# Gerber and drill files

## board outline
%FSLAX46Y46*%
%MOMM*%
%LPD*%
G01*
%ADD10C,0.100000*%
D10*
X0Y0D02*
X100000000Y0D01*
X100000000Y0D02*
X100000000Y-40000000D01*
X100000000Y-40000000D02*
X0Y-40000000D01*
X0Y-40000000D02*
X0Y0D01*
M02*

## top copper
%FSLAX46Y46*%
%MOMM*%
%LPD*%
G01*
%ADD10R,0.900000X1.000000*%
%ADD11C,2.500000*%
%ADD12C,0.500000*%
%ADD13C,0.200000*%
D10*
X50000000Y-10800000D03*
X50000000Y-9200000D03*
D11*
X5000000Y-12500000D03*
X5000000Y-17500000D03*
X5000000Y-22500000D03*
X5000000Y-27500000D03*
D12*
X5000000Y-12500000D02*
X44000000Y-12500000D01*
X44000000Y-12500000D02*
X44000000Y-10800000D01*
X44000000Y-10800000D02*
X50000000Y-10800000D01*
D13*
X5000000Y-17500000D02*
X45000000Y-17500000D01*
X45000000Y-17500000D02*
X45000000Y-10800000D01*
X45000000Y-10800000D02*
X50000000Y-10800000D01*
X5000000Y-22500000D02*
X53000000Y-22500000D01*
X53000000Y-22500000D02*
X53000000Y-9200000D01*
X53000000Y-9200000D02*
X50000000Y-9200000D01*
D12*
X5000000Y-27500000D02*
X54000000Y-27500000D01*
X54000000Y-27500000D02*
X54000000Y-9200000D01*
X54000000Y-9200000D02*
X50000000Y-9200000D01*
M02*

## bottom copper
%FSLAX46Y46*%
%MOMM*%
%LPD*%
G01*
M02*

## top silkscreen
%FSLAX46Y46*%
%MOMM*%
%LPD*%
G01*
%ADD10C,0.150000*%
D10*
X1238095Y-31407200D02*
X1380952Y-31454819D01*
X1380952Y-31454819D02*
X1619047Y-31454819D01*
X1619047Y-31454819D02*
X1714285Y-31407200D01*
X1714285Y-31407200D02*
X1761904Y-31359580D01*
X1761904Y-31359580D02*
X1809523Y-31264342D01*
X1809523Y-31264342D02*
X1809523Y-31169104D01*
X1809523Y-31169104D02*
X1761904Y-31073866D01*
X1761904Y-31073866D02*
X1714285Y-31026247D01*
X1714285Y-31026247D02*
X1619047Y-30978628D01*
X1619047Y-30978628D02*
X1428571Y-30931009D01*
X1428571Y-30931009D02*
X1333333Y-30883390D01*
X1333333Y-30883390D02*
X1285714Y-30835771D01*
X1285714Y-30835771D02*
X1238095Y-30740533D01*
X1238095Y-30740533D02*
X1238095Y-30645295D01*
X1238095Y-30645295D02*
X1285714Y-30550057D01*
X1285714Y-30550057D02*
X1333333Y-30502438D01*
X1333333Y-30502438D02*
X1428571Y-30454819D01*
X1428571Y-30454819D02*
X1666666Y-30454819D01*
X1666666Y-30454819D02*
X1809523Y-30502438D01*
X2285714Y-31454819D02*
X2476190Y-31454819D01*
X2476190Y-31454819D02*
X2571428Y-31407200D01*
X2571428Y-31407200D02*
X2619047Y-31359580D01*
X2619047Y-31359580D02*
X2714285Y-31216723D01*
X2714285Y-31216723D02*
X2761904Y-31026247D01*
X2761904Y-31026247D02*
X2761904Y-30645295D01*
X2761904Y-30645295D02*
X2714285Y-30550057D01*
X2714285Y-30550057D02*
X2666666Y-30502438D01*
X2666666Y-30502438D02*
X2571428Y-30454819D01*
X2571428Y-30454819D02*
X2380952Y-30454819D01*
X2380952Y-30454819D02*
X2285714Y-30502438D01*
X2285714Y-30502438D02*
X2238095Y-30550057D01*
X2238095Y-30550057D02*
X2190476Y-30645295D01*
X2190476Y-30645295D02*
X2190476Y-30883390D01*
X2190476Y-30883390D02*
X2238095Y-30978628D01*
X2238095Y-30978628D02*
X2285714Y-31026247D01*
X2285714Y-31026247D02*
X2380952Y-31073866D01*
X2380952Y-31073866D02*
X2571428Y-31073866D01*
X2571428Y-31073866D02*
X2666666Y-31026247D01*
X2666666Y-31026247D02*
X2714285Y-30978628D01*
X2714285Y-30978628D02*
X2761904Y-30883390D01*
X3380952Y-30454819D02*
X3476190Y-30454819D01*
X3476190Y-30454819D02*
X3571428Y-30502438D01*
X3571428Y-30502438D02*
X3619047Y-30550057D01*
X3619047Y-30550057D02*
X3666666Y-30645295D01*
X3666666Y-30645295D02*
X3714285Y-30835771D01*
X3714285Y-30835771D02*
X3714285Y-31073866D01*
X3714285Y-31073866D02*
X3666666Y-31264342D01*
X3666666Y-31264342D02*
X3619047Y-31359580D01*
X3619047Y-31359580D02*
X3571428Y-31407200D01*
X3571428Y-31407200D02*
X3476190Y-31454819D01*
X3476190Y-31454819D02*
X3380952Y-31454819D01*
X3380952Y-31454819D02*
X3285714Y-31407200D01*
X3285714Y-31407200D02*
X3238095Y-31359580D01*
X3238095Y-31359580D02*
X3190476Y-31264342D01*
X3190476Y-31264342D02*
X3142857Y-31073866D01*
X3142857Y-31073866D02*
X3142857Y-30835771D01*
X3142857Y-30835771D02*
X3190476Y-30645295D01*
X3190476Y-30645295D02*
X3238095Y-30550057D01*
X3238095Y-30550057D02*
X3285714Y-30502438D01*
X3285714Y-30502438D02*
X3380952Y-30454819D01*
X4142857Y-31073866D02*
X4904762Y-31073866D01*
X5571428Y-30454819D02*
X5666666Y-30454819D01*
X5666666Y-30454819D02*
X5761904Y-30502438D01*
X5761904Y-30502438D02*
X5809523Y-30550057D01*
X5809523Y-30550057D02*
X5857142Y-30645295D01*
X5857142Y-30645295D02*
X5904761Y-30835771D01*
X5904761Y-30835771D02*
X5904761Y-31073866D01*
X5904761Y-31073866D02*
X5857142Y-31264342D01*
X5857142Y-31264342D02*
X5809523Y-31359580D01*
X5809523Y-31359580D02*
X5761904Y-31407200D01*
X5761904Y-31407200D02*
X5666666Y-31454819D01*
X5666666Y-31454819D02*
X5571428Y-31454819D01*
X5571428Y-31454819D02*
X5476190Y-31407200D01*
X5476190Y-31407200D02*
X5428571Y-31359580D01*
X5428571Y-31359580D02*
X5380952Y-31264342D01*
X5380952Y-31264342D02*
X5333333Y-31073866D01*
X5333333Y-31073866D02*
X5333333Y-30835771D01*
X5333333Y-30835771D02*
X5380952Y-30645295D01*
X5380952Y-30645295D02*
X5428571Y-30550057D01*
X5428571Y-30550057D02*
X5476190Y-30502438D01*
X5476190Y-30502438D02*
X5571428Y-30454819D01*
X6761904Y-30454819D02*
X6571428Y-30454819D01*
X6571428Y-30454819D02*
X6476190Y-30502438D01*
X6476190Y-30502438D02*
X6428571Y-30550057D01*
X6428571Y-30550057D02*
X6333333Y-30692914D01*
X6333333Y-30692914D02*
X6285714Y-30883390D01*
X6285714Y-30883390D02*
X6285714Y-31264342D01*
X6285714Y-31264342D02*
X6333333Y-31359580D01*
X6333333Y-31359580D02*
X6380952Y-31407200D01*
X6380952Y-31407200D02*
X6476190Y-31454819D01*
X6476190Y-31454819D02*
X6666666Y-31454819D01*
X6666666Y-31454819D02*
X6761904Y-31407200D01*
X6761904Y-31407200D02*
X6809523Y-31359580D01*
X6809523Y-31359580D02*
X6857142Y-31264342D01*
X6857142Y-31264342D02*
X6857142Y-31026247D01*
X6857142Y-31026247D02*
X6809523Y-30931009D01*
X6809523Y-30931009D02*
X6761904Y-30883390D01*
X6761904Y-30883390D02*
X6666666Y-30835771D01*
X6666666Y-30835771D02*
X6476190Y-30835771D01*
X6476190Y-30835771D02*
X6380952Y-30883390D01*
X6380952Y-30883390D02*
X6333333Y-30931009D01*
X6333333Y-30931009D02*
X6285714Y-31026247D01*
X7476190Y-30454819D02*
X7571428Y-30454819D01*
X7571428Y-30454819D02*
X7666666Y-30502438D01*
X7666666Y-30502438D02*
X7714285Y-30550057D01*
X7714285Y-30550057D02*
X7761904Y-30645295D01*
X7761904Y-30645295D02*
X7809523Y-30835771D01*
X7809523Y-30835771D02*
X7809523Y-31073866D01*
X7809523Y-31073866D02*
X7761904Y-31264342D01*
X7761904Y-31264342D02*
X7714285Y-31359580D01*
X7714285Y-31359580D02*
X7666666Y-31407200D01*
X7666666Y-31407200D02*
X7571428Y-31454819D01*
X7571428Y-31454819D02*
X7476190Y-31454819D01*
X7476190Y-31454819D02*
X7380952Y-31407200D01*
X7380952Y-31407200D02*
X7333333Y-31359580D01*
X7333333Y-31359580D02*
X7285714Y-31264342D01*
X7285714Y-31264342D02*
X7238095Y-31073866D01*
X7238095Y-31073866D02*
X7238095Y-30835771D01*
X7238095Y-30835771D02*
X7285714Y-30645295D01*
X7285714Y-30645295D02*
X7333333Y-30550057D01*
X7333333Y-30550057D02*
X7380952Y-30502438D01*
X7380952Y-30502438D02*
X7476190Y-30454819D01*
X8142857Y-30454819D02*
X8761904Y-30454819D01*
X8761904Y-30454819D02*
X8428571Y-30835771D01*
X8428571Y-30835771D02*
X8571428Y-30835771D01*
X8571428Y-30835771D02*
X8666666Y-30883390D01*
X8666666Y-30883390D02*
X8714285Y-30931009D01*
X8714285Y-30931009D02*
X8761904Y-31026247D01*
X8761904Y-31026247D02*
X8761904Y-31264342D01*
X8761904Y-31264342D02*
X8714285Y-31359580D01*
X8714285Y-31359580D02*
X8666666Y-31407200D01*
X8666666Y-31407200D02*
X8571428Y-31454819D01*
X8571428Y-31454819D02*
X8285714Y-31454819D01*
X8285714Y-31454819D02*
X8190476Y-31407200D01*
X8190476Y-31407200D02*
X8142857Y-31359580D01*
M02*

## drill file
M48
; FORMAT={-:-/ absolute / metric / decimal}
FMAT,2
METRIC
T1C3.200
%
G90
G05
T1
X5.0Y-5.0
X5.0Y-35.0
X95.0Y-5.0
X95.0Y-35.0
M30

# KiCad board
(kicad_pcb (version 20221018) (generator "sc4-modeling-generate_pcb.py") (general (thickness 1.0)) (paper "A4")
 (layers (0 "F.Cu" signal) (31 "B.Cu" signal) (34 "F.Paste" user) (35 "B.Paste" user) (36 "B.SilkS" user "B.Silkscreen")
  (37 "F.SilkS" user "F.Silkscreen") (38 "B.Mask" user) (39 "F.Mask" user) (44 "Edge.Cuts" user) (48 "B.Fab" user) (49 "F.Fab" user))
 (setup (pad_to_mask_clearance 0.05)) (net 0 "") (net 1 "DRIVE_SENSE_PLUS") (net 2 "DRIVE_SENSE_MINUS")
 (gr_line (start 0.0 0.0) (end 100.0 0.0) (layer "Edge.Cuts") (width 0.1))
 (gr_line (start 100.0 0.0) (end 100.0 40.0) (layer "Edge.Cuts") (width 0.1))
 (gr_line (start 100.0 40.0) (end 0.0 40.0) (layer "Edge.Cuts") (width 0.1))
 (gr_line (start 0.0 40.0) (end 0.0 0.0) (layer "Edge.Cuts") (width 0.1))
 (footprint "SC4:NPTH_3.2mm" (layer "F.Cu") (at 5.0 5.0)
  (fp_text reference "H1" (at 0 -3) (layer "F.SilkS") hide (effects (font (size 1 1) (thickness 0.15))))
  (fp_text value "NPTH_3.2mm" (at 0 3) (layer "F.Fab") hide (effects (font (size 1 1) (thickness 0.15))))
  (pad "1" np_thru_hole circle (at 0 0) (size 3.2 3.2) (drill 3.2) (layers "*.Cu" "*.Mask")))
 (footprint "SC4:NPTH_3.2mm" (layer "F.Cu") (at 95.0 5.0)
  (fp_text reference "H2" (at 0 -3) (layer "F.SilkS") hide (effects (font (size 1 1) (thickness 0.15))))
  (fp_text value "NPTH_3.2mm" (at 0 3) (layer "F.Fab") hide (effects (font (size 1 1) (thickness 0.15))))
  (pad "1" np_thru_hole circle (at 0 0) (size 3.2 3.2) (drill 3.2) (layers "*.Cu" "*.Mask")))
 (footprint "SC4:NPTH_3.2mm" (layer "F.Cu") (at 5.0 35.0)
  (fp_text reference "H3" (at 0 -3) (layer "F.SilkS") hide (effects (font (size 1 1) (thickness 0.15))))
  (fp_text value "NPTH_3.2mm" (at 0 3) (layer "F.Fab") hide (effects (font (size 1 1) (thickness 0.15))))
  (pad "1" np_thru_hole circle (at 0 0) (size 3.2 3.2) (drill 3.2) (layers "*.Cu" "*.Mask")))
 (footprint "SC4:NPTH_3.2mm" (layer "F.Cu") (at 95.0 35.0)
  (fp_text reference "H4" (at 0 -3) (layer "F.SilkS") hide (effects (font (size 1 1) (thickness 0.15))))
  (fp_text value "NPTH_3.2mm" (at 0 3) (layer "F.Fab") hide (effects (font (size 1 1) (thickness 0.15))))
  (pad "1" np_thru_hole circle (at 0 0) (size 3.2 3.2) (drill 3.2) (layers "*.Cu" "*.Mask")))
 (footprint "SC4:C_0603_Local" (layer "F.Cu") (at 50.0 10.0 90)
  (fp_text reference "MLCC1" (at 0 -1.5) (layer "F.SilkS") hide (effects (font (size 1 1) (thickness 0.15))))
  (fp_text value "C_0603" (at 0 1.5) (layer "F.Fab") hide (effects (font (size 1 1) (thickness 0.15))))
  (pad "1" smd rect (at -0.8 0) (size 0.9 1.0) (layers "F.Cu" "F.Paste" "F.Mask") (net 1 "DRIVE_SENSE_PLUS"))
  (pad "2" smd rect (at 0.8 0) (size 0.9 1.0) (layers "F.Cu" "F.Paste" "F.Mask") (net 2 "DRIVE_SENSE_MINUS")))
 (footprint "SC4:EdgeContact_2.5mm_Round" (layer "F.Cu") (at 5.0 12.5)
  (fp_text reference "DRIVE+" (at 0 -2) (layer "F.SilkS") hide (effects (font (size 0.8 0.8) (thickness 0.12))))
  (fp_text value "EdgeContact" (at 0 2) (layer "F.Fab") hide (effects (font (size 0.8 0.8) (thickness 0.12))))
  (pad "1" smd circle (at 0 0) (size 2.5 2.5) (layers "F.Cu" "F.Mask") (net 1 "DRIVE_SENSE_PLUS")))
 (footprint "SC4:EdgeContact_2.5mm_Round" (layer "F.Cu") (at 5.0 17.5)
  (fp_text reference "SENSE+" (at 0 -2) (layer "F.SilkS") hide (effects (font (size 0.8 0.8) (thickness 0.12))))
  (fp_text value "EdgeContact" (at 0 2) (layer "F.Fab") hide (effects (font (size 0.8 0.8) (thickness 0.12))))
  (pad "1" smd circle (at 0 0) (size 2.5 2.5) (layers "F.Cu" "F.Mask") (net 1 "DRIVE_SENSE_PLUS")))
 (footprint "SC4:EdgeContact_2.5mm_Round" (layer "F.Cu") (at 5.0 22.5)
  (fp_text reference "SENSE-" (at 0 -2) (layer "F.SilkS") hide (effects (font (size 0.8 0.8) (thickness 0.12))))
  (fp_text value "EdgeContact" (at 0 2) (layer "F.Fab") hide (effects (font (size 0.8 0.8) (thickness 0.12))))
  (pad "1" smd circle (at 0 0) (size 2.5 2.5) (layers "F.Cu" "F.Mask") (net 2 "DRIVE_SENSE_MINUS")))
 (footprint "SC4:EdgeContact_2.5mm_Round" (layer "F.Cu") (at 5.0 27.5)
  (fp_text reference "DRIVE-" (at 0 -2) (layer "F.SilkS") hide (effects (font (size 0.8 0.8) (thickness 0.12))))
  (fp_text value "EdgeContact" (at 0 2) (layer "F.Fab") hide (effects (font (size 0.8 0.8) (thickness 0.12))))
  (pad "1" smd circle (at 0 0) (size 2.5 2.5) (layers "F.Cu" "F.Mask") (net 2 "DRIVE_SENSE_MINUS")))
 (segment (start 5.0 12.5) (end 44.0 12.5) (width 0.5) (layer "F.Cu") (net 1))
 (segment (start 44.0 12.5) (end 44.0 10.8) (width 0.5) (layer "F.Cu") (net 1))
 (segment (start 44.0 10.8) (end 50.0 10.8) (width 0.5) (layer "F.Cu") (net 1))
 (segment (start 5.0 17.5) (end 45.0 17.5) (width 0.2) (layer "F.Cu") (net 1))
 (segment (start 45.0 17.5) (end 45.0 10.8) (width 0.2) (layer "F.Cu") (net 1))
 (segment (start 45.0 10.8) (end 50.0 10.8) (width 0.2) (layer "F.Cu") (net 1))
 (segment (start 5.0 22.5) (end 53.0 22.5) (width 0.2) (layer "F.Cu") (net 2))
 (segment (start 53.0 22.5) (end 53.0 9.2) (width 0.2) (layer "F.Cu") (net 2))
 (segment (start 53.0 9.2) (end 50.0 9.2) (width 0.2) (layer "F.Cu") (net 2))
 (segment (start 5.0 27.5) (end 54.0 27.5) (width 0.5) (layer "F.Cu") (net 2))
 (segment (start 54.0 27.5) (end 54.0 9.2) (width 0.5) (layer "F.Cu") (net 2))
 (segment (start 54.0 9.2) (end 50.0 9.2) (width 0.5) (layer "F.Cu") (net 2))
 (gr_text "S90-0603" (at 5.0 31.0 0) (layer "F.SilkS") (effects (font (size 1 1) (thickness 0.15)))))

